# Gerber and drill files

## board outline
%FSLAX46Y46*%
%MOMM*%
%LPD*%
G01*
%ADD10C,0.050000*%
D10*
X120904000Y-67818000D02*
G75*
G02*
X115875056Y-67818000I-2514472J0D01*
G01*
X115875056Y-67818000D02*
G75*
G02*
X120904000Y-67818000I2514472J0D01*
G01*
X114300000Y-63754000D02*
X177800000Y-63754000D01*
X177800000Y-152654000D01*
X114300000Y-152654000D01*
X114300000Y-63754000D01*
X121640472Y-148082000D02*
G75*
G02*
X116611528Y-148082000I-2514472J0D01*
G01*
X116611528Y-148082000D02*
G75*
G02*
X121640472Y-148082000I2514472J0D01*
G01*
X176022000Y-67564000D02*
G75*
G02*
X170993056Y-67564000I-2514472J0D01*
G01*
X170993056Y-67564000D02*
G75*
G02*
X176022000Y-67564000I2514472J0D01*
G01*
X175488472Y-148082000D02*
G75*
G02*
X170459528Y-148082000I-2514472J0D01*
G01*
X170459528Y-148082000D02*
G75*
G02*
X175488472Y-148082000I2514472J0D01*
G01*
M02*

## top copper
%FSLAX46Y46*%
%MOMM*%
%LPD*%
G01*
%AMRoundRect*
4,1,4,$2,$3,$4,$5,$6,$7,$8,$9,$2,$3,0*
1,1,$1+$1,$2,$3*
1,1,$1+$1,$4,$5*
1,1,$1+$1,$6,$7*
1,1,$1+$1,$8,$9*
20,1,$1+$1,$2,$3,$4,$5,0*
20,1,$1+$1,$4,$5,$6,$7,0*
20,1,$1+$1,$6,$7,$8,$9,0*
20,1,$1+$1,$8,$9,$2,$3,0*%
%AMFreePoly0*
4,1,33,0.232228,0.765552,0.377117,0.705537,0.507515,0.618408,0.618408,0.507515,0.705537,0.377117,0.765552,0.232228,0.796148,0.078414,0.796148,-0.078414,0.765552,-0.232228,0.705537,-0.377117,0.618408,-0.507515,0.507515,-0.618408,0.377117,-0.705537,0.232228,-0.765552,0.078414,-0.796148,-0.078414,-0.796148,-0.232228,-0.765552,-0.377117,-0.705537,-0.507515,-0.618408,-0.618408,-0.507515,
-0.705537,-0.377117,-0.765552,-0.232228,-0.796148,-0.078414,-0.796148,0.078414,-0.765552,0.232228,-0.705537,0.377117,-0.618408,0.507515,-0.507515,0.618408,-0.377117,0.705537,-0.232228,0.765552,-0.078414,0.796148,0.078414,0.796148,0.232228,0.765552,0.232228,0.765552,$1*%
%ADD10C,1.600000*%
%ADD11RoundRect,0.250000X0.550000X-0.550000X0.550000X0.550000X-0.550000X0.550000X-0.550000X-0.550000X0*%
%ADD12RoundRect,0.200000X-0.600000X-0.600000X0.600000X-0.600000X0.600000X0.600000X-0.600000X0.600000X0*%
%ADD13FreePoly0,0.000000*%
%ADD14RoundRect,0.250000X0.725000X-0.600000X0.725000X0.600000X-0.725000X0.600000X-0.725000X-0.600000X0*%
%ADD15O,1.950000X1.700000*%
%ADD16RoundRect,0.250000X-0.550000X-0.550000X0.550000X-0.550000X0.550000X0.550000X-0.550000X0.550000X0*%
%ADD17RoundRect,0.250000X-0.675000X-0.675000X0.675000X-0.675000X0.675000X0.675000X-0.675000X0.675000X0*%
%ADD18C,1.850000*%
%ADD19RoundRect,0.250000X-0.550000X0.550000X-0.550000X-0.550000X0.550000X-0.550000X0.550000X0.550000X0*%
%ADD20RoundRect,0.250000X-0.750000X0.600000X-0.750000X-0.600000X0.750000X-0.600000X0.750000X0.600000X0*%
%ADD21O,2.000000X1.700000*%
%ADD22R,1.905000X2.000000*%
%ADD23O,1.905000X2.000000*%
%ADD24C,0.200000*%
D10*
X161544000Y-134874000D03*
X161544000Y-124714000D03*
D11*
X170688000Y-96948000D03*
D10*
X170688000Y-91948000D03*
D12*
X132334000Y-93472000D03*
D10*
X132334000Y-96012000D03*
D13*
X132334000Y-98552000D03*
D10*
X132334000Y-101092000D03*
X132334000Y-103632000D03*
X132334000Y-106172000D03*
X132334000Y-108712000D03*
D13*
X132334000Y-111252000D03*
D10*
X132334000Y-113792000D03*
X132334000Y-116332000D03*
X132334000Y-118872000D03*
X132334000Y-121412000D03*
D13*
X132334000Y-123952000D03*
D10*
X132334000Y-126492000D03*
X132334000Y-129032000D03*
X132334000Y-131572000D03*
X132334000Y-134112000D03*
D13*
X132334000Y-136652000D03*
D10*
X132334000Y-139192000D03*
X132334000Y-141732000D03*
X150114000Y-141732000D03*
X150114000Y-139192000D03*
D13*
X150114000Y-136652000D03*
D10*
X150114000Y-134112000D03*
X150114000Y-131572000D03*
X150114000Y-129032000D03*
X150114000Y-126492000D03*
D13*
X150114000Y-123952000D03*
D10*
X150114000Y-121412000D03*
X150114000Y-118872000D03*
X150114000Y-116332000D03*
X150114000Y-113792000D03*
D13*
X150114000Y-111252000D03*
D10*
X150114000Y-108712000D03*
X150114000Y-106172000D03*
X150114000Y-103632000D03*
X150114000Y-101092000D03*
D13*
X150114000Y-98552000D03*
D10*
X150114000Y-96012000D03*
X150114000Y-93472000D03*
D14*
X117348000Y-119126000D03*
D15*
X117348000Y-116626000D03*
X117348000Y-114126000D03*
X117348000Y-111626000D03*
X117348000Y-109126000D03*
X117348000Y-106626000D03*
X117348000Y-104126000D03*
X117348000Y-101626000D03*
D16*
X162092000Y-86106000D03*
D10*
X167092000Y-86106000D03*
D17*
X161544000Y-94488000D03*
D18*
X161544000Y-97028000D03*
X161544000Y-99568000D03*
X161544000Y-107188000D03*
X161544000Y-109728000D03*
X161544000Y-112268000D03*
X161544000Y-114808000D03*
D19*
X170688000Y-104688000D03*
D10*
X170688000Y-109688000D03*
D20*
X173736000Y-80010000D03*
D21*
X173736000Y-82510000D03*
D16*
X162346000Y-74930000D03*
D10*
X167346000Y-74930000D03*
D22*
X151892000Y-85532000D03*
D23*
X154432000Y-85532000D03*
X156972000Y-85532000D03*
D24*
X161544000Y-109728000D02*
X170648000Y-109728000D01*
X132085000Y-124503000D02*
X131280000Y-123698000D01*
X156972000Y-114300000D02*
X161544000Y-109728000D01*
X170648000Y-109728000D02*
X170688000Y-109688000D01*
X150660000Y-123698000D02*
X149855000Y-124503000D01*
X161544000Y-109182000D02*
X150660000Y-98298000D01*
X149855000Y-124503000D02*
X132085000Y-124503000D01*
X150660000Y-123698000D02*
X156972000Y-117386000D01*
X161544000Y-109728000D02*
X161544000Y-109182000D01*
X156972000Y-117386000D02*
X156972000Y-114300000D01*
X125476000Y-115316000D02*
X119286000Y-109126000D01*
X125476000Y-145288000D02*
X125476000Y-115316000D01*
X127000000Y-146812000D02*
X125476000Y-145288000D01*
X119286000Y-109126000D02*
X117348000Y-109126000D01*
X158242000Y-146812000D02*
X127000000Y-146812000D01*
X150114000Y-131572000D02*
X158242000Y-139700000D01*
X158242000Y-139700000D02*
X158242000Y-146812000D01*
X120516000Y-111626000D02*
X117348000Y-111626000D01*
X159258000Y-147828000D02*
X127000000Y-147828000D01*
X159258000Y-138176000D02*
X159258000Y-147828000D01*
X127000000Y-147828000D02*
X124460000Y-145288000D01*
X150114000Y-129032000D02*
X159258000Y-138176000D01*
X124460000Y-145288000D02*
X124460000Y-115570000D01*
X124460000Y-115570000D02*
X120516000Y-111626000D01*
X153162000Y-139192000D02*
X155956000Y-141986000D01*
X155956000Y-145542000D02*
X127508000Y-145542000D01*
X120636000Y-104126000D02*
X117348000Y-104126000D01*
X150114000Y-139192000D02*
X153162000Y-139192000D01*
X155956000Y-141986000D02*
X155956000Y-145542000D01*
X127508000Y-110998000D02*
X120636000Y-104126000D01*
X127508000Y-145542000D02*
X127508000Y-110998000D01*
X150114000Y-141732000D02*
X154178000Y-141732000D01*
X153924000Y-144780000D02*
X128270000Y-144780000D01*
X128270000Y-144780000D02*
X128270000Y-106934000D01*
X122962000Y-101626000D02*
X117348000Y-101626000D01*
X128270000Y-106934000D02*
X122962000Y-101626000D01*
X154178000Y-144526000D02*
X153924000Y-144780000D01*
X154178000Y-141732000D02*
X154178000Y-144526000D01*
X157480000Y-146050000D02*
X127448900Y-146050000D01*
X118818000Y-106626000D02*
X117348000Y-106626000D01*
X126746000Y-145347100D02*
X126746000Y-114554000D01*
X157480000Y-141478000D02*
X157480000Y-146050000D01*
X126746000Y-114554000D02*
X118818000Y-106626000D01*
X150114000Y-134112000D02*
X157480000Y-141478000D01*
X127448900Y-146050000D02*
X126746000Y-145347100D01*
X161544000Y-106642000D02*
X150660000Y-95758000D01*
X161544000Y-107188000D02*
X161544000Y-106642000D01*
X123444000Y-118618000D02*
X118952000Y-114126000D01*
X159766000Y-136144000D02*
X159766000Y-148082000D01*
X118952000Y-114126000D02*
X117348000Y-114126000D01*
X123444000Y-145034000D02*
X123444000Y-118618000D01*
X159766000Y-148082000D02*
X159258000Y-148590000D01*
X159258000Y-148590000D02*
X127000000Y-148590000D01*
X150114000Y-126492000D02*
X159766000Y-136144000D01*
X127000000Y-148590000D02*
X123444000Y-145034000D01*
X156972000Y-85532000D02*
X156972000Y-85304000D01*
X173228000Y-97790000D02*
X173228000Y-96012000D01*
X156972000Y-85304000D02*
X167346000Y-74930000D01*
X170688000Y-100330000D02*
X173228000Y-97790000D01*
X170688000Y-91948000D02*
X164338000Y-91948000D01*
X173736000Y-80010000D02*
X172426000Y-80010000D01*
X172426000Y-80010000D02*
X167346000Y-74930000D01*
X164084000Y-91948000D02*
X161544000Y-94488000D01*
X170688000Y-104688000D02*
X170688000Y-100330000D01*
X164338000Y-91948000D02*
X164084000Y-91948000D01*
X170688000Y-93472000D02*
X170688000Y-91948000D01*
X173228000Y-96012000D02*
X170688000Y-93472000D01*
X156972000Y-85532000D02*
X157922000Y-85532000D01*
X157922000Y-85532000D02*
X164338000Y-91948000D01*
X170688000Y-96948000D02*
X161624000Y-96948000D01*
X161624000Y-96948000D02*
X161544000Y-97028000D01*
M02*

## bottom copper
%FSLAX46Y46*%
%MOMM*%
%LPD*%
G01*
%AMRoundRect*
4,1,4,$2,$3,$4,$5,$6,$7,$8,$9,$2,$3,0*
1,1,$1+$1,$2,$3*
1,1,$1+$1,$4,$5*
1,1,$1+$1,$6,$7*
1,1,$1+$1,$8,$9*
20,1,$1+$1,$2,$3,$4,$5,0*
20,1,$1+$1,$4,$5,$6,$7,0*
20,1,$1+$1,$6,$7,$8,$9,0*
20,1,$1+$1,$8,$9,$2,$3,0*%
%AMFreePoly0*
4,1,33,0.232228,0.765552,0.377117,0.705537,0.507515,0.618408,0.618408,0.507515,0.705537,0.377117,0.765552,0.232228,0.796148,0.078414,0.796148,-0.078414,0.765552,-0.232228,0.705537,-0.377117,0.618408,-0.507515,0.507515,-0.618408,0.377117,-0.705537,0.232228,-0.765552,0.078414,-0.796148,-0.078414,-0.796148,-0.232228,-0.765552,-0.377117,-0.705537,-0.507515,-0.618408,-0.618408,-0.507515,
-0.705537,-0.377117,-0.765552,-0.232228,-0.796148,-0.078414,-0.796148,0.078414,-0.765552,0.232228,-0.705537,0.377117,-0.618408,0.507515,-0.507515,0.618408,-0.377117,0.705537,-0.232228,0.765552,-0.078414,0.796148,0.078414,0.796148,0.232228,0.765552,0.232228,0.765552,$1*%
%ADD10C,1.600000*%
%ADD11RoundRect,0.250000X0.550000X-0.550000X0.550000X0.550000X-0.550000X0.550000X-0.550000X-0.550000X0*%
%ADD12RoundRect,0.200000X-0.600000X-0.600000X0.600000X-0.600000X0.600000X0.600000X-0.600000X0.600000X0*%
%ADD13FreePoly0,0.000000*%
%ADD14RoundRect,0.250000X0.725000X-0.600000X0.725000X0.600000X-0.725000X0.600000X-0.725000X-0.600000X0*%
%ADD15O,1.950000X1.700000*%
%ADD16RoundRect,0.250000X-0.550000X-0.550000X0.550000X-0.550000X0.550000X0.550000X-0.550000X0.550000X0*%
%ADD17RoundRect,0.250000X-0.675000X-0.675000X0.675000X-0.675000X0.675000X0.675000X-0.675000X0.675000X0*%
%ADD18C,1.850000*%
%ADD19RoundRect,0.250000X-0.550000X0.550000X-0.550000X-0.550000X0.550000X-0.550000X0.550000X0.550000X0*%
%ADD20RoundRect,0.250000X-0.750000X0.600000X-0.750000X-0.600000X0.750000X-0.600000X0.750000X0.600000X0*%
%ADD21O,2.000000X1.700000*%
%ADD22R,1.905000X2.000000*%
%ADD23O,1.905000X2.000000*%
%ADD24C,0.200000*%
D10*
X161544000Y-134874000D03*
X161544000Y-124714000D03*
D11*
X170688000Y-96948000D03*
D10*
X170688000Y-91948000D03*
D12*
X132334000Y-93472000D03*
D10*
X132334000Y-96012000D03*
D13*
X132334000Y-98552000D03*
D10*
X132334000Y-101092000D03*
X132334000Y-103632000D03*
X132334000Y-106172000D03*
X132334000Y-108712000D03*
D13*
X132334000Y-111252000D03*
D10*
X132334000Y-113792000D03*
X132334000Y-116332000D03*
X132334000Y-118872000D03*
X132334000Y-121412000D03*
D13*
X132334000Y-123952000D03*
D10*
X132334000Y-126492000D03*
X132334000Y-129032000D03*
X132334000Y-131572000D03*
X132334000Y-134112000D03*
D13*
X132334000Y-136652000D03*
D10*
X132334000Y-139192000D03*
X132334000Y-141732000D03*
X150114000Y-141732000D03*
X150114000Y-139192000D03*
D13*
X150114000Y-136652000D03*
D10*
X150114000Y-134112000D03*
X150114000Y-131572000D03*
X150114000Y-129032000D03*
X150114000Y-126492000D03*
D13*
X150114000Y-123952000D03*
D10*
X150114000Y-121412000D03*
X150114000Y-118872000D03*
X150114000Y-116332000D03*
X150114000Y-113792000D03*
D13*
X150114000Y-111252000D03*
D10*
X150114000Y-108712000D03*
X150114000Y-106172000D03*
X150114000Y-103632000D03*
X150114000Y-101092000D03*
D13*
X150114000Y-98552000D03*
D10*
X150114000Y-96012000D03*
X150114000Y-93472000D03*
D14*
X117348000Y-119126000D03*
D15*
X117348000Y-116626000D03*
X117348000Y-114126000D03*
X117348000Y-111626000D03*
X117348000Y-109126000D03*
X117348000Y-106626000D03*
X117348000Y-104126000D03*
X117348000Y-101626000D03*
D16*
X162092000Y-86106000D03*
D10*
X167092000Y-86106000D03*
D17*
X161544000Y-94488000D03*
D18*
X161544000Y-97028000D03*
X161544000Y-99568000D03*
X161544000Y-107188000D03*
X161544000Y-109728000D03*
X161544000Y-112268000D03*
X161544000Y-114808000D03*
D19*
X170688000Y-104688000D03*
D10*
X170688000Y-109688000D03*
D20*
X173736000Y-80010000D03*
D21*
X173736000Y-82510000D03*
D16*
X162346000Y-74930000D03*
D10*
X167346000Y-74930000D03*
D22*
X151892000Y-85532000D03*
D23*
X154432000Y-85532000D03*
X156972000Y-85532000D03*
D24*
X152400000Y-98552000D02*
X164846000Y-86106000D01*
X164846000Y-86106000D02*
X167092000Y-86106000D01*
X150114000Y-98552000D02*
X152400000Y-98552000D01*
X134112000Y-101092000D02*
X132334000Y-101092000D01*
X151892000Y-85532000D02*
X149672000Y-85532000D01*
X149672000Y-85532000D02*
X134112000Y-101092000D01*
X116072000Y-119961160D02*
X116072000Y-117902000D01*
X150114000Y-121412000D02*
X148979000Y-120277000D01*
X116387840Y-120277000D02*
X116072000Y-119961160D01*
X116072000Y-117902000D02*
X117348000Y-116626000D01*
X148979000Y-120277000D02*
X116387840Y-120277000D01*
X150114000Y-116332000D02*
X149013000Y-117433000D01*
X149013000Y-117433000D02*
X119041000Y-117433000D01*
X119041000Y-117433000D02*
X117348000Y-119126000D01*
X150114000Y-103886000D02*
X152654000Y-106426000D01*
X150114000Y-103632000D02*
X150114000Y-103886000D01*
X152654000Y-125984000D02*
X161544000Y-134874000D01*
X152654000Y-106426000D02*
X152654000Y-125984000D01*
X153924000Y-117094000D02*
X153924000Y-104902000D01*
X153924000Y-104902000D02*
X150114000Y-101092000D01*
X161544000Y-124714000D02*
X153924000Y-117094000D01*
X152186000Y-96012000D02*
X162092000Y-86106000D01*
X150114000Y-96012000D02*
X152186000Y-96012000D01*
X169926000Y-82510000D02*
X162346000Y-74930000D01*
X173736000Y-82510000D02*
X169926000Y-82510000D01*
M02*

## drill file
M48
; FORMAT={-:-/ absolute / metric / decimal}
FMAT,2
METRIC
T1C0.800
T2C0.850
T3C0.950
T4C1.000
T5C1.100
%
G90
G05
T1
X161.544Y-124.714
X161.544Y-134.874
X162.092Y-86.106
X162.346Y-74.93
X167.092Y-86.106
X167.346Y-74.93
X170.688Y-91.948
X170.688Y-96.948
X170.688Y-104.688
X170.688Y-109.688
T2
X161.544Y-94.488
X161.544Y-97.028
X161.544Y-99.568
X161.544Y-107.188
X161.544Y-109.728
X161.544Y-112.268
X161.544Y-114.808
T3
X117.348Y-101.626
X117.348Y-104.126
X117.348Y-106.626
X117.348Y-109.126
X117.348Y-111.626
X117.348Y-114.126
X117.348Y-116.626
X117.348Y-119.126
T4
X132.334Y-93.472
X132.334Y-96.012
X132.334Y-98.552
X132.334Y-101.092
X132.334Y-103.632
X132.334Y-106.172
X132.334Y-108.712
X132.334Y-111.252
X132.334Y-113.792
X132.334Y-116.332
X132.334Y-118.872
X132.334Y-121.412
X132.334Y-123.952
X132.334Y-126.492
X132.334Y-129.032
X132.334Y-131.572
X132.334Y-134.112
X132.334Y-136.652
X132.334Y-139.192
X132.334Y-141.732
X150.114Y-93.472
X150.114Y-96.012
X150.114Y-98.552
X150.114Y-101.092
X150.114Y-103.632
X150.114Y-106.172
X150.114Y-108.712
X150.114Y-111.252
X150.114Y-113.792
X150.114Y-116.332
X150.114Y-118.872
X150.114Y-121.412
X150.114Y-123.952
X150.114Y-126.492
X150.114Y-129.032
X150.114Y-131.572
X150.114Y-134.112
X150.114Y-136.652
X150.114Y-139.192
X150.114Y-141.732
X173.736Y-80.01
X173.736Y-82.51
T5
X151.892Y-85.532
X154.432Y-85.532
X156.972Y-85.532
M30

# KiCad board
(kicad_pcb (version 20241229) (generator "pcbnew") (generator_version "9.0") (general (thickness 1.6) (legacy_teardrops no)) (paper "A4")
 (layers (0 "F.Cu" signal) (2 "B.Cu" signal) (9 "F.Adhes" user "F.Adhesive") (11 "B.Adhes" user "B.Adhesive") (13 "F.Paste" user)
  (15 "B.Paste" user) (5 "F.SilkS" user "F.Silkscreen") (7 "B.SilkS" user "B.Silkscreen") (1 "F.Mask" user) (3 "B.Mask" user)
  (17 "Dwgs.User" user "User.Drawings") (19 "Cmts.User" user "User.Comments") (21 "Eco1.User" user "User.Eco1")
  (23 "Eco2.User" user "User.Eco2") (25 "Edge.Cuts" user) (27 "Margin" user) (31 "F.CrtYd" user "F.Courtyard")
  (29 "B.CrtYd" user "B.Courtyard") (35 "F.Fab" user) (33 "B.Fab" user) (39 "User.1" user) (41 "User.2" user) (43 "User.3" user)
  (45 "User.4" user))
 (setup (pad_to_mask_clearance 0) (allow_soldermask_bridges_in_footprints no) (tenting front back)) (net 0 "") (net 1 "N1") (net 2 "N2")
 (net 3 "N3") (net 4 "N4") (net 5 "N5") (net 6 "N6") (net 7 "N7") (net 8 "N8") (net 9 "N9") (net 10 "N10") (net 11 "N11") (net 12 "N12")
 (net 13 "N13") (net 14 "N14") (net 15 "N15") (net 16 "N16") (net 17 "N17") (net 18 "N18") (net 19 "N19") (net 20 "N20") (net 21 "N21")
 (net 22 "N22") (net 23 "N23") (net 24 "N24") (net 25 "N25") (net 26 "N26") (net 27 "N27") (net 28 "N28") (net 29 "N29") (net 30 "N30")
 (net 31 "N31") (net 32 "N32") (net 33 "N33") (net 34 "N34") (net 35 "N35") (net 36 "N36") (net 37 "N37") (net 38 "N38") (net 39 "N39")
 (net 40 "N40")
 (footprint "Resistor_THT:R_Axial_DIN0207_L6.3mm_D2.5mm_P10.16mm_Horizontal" (layer "F.Cu") (at 161.544 134.874 90)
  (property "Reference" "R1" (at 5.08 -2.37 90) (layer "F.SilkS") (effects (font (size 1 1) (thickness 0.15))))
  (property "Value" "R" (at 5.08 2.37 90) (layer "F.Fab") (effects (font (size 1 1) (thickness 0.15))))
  (pad "1" thru_hole circle (at 0 0 90) (size 1.6 1.6) (drill 0.8) (layers "*.Cu" "*.Mask") (remove_unused_layers no) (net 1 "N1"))
  (pad "2" thru_hole circle (at 10.16 0 90) (size 1.6 1.6) (drill 0.8) (layers "*.Cu" "*.Mask") (remove_unused_layers no) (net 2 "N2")))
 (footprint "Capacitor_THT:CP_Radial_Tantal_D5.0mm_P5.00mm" (layer "F.Cu") (at 170.688 96.948 90)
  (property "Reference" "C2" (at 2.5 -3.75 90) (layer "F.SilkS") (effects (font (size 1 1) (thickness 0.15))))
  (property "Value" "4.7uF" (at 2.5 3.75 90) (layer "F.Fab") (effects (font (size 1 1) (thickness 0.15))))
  (pad "1" thru_hole roundrect (at 0 0 90) (size 1.6 1.6) (drill 0.8) (layers "*.Cu" "*.Mask") (remove_unused_layers no)
   (roundrect_rratio 0.15625) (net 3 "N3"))
  (pad "2" thru_hole circle (at 5 0 90) (size 1.6 1.6) (drill 0.8) (layers "*.Cu" "*.Mask") (remove_unused_layers no) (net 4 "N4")))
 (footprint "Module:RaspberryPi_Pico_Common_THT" (layer "F.Cu") (at 132.334 93.472)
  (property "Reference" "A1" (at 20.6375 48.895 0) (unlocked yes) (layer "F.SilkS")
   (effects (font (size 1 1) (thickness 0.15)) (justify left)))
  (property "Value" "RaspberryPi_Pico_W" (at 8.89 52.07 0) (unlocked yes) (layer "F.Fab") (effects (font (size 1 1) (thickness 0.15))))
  (pad "1" thru_hole roundrect (at 0 0) (size 1.6 1.6) (drill 1) (layers "*.Cu" "*.Mask") (remove_unused_layers no) (roundrect_rratio 0.125)
   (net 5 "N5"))
  (pad "2" thru_hole circle (at 0 2.54) (size 1.6 1.6) (drill 1) (layers "*.Cu" "*.Mask") (remove_unused_layers no) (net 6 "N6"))
  (pad "3" thru_hole custom (at 0 5.08) (size 1.6 1.6) (drill 1) (layers "*.Cu" "*.Mask") (remove_unused_layers no) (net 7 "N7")
   (options (clearance outline) (anchor circle)) (primitives))
  (pad "4" thru_hole circle (at 0 7.62) (size 1.6 1.6) (drill 1) (layers "*.Cu" "*.Mask") (remove_unused_layers no) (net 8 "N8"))
  (pad "5" thru_hole circle (at 0 10.16) (size 1.6 1.6) (drill 1) (layers "*.Cu" "*.Mask") (remove_unused_layers no) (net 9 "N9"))
  (pad "6" thru_hole circle (at 0 12.7) (size 1.6 1.6) (drill 1) (layers "*.Cu" "*.Mask") (remove_unused_layers no) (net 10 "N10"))
  (pad "7" thru_hole circle (at 0 15.24) (size 1.6 1.6) (drill 1) (layers "*.Cu" "*.Mask") (remove_unused_layers no) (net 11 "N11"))
  (pad "8" thru_hole custom (at 0 17.78) (size 1.6 1.6) (drill 1) (layers "*.Cu" "*.Mask") (remove_unused_layers no) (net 7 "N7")
   (options (clearance outline) (anchor circle)) (primitives))
  (pad "9" thru_hole circle (at 0 20.32) (size 1.6 1.6) (drill 1) (layers "*.Cu" "*.Mask") (remove_unused_layers no) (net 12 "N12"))
  (pad "10" thru_hole circle (at 0 22.86) (size 1.6 1.6) (drill 1) (layers "*.Cu" "*.Mask") (remove_unused_layers no) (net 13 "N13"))
  (pad "11" thru_hole circle (at 0 25.4) (size 1.6 1.6) (drill 1) (layers "*.Cu" "*.Mask") (remove_unused_layers no) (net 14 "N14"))
  (pad "12" thru_hole circle (at 0 27.94) (size 1.6 1.6) (drill 1) (layers "*.Cu" "*.Mask") (remove_unused_layers no) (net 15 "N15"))
  (pad "13" thru_hole custom (at 0 30.48) (size 1.6 1.6) (drill 1) (layers "*.Cu" "*.Mask") (remove_unused_layers no) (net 7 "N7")
   (options (clearance outline) (anchor circle)) (primitives))
  (pad "14" thru_hole circle (at 0 33.02) (size 1.6 1.6) (drill 1) (layers "*.Cu" "*.Mask") (remove_unused_layers no) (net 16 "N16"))
  (pad "15" thru_hole circle (at 0 35.56) (size 1.6 1.6) (drill 1) (layers "*.Cu" "*.Mask") (remove_unused_layers no) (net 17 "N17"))
  (pad "16" thru_hole circle (at 0 38.1) (size 1.6 1.6) (drill 1) (layers "*.Cu" "*.Mask") (remove_unused_layers no) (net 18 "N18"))
  (pad "17" thru_hole circle (at 0 40.64) (size 1.6 1.6) (drill 1) (layers "*.Cu" "*.Mask") (remove_unused_layers no) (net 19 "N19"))
  (pad "18" thru_hole custom (at 0 43.18) (size 1.6 1.6) (drill 1) (layers "*.Cu" "*.Mask") (remove_unused_layers no) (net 7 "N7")
   (options (clearance outline) (anchor circle)) (primitives))
  (pad "19" thru_hole circle (at 0 45.72) (size 1.6 1.6) (drill 1) (layers "*.Cu" "*.Mask") (remove_unused_layers no) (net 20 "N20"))
  (pad "20" thru_hole circle (at 0 48.26) (size 1.6 1.6) (drill 1) (layers "*.Cu" "*.Mask") (remove_unused_layers no) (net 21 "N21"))
  (pad "21" thru_hole circle (at 17.78 48.26) (size 1.6 1.6) (drill 1) (layers "*.Cu" "*.Mask") (remove_unused_layers no) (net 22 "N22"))
  (pad "22" thru_hole circle (at 17.78 45.72) (size 1.6 1.6) (drill 1) (layers "*.Cu" "*.Mask") (remove_unused_layers no) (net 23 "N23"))
  (pad "23" thru_hole custom (at 17.78 43.18) (size 1.6 1.6) (drill 1) (layers "*.Cu" "*.Mask") (remove_unused_layers no) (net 7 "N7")
   (options (clearance outline) (anchor circle)) (primitives))
  (pad "24" thru_hole circle (at 17.78 40.64) (size 1.6 1.6) (drill 1) (layers "*.Cu" "*.Mask") (remove_unused_layers no) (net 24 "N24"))
  (pad "25" thru_hole circle (at 17.78 38.1) (size 1.6 1.6) (drill 1) (layers "*.Cu" "*.Mask") (remove_unused_layers no) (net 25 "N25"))
  (pad "26" thru_hole circle (at 17.78 35.56) (size 1.6 1.6) (drill 1) (layers "*.Cu" "*.Mask") (remove_unused_layers no) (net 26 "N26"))
  (pad "27" thru_hole circle (at 17.78 33.02) (size 1.6 1.6) (drill 1) (layers "*.Cu" "*.Mask") (remove_unused_layers no) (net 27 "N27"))
  (pad "28" thru_hole custom (at 17.78 30.48) (size 1.6 1.6) (drill 1) (layers "*.Cu" "*.Mask") (remove_unused_layers no) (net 7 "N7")
   (options (clearance outline) (anchor circle)) (primitives))
  (pad "29" thru_hole circle (at 17.78 27.94) (size 1.6 1.6) (drill 1) (layers "*.Cu" "*.Mask") (remove_unused_layers no) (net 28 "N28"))
  (pad "30" thru_hole circle (at 17.78 25.4) (size 1.6 1.6) (drill 1) (layers "*.Cu" "*.Mask") (remove_unused_layers no) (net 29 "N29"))
  (pad "31" thru_hole circle (at 17.78 22.86) (size 1.6 1.6) (drill 1) (layers "*.Cu" "*.Mask") (remove_unused_layers no) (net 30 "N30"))
  (pad "32" thru_hole circle (at 17.78 20.32) (size 1.6 1.6) (drill 1) (layers "*.Cu" "*.Mask") (remove_unused_layers no) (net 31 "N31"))
  (pad "33" thru_hole custom (at 17.78 17.78) (size 1.6 1.6) (drill 1) (layers "*.Cu" "*.Mask") (remove_unused_layers no) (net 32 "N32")
   (options (clearance outline) (anchor circle)) (primitives))
  (pad "34" thru_hole circle (at 17.78 15.24) (size 1.6 1.6) (drill 1) (layers "*.Cu" "*.Mask") (remove_unused_layers no) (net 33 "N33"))
  (pad "35" thru_hole circle (at 17.78 12.7) (size 1.6 1.6) (drill 1) (layers "*.Cu" "*.Mask") (remove_unused_layers no) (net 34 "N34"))
  (pad "36" thru_hole circle (at 17.78 10.16) (size 1.6 1.6) (drill 1) (layers "*.Cu" "*.Mask") (remove_unused_layers no) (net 1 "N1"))
  (pad "37" thru_hole circle (at 17.78 7.62) (size 1.6 1.6) (drill 1) (layers "*.Cu" "*.Mask") (remove_unused_layers no) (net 2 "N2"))
  (pad "38" thru_hole custom (at 17.78 5.08) (size 1.6 1.6) (drill 1) (layers "*.Cu" "*.Mask") (remove_unused_layers no) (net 7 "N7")
   (options (clearance outline) (anchor circle)) (primitives))
  (pad "39" thru_hole circle (at 17.78 2.54) (size 1.6 1.6) (drill 1) (layers "*.Cu" "*.Mask") (remove_unused_layers no) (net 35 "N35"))
  (pad "40" thru_hole circle (at 17.78 0) (size 1.6 1.6) (drill 1) (layers "*.Cu" "*.Mask") (remove_unused_layers no) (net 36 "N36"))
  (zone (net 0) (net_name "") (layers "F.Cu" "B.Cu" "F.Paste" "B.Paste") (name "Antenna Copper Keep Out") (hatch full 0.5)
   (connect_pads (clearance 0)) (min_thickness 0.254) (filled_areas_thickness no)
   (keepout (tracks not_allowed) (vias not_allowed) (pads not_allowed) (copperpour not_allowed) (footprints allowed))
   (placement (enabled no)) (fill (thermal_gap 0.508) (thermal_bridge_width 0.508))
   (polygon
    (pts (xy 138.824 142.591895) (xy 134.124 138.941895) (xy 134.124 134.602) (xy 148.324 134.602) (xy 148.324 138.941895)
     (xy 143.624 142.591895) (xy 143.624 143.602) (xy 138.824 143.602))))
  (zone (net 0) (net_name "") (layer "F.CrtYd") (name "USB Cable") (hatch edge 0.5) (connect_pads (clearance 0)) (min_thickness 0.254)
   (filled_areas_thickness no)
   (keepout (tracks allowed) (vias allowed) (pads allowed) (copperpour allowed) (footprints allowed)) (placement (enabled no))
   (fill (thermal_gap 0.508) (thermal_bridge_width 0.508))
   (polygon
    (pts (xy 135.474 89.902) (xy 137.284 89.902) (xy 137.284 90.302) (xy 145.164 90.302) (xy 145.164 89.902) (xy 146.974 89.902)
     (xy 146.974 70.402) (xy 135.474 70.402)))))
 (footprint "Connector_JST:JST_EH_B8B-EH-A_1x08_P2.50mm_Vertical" (layer "F.Cu") (at 117.348 119.126 90)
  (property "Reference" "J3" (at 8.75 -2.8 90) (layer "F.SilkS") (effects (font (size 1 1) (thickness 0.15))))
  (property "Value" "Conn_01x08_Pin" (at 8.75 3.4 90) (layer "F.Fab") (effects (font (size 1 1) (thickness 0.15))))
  (pad "1" thru_hole roundrect (at 0 0 90) (size 1.7 1.95) (drill 0.95) (layers "*.Cu" "*.Mask") (remove_unused_layers no)
   (roundrect_rratio 0.147059) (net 30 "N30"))
  (pad "2" thru_hole oval (at 2.5 0 90) (size 1.7 1.95) (drill 0.95) (layers "*.Cu" "*.Mask") (remove_unused_layers no) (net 28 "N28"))
  (pad "3" thru_hole oval (at 5 0 90) (size 1.7 1.95) (drill 0.95) (layers "*.Cu" "*.Mask") (remove_unused_layers no) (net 27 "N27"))
  (pad "4" thru_hole oval (at 7.5 0 90) (size 1.7 1.95) (drill 0.95) (layers "*.Cu" "*.Mask") (remove_unused_layers no) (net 26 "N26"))
  (pad "5" thru_hole oval (at 10 0 90) (size 1.7 1.95) (drill 0.95) (layers "*.Cu" "*.Mask") (remove_unused_layers no) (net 25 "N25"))
  (pad "6" thru_hole oval (at 12.5 0 90) (size 1.7 1.95) (drill 0.95) (layers "*.Cu" "*.Mask") (remove_unused_layers no) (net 24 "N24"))
  (pad "7" thru_hole oval (at 15 0 90) (size 1.7 1.95) (drill 0.95) (layers "*.Cu" "*.Mask") (remove_unused_layers no) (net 23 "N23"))
  (pad "8" thru_hole oval (at 17.5 0 90) (size 1.7 1.95) (drill 0.95) (layers "*.Cu" "*.Mask") (remove_unused_layers no) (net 22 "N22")))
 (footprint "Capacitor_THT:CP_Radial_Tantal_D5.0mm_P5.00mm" (layer "F.Cu") (at 162.092 86.106)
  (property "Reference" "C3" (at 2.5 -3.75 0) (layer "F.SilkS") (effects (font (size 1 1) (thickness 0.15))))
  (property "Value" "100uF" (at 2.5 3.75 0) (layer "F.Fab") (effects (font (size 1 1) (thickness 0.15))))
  (pad "1" thru_hole roundrect (at 0 0) (size 1.6 1.6) (drill 0.8) (layers "*.Cu" "*.Mask") (remove_unused_layers no)
   (roundrect_rratio 0.15625) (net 35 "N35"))
  (pad "2" thru_hole circle (at 5 0) (size 1.6 1.6) (drill 0.8) (layers "*.Cu" "*.Mask") (remove_unused_layers no) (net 7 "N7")))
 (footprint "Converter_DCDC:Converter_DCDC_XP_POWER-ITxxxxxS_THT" (layer "F.Cu") (at 161.544 94.488)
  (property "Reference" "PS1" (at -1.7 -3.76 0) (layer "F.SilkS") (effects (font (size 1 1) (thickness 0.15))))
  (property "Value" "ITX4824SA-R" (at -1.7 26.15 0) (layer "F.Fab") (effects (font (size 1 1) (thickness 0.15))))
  (pad "1" thru_hole roundrect (at 0 0) (size 1.85 1.85) (drill 0.85) (layers "*.Cu" "*.Mask") (remove_unused_layers no)
   (roundrect_rratio 0.135135) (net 4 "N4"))
  (pad "2" thru_hole circle (at 0 2.54) (size 1.85 1.85) (drill 0.85) (layers "*.Cu" "*.Mask") (remove_unused_layers no) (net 3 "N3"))
  (pad "3" thru_hole circle (at 0 5.08) (size 1.85 1.85) (drill 0.85) (layers "*.Cu" "*.Mask") (remove_unused_layers no) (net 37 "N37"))
  (pad "6" thru_hole circle (at 0 12.7) (size 1.85 1.85) (drill 0.85) (layers "*.Cu" "*.Mask") (remove_unused_layers no) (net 35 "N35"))
  (pad "7" thru_hole circle (at 0 15.24) (size 1.85 1.85) (drill 0.85) (layers "*.Cu" "*.Mask") (remove_unused_layers no) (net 7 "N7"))
  (pad "8" thru_hole circle (at 0 17.78) (size 1.85 1.85) (drill 0.85) (layers "*.Cu" "*.Mask") (remove_unused_layers no) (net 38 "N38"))
  (pad "9" thru_hole circle (at 0 20.32) (size 1.85 1.85) (drill 0.85) (layers "*.Cu" "*.Mask") (remove_unused_layers no)))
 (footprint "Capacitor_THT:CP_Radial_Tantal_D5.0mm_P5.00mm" (layer "F.Cu") (at 170.688 104.688 -90)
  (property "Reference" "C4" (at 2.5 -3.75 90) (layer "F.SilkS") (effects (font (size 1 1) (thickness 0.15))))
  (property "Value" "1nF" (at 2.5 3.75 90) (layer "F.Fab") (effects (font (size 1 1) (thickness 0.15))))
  (pad "1" thru_hole roundrect (at 0 0 270) (size 1.6 1.6) (drill 0.8) (layers "*.Cu" "*.Mask") (remove_unused_layers no)
   (roundrect_rratio 0.15625) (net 4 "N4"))
  (pad "2" thru_hole circle (at 5 0 270) (size 1.6 1.6) (drill 0.8) (layers "*.Cu" "*.Mask") (remove_unused_layers no) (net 7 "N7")))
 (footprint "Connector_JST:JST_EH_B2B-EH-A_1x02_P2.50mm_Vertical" (layer "F.Cu") (at 173.736 80.01 -90)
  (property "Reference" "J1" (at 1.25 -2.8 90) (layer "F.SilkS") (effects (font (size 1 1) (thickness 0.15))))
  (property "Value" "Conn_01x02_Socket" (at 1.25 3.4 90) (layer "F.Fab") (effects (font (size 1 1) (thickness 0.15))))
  (pad "1" thru_hole roundrect (at 0 0 270) (size 1.7 2) (drill 1) (layers "*.Cu" "*.Mask") (remove_unused_layers no)
   (roundrect_rratio 0.147059) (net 4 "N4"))
  (pad "2" thru_hole oval (at 2.5 0 270) (size 1.7 2) (drill 1) (layers "*.Cu" "*.Mask") (remove_unused_layers no) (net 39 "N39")))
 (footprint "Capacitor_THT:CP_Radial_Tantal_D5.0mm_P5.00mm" (layer "F.Cu") (at 162.346 74.93)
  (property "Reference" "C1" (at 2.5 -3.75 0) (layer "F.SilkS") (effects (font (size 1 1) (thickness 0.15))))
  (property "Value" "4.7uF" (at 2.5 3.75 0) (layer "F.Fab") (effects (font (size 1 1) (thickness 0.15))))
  (pad "1" thru_hole roundrect (at 0 0) (size 1.6 1.6) (drill 0.8) (layers "*.Cu" "*.Mask") (remove_unused_layers no)
   (roundrect_rratio 0.15625) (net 39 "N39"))
  (pad "2" thru_hole circle (at 5 0) (size 1.6 1.6) (drill 0.8) (layers "*.Cu" "*.Mask") (remove_unused_layers no) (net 4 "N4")))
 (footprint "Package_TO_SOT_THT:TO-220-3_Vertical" (layer "F.Cu") (at 151.892 85.532)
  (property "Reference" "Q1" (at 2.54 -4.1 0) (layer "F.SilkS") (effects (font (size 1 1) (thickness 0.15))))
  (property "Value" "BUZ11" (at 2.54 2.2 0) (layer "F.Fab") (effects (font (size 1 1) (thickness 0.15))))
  (pad "1" thru_hole rect (at 0 0) (size 1.905 2) (drill 1.1) (layers "*.Cu" "*.Mask") (remove_unused_layers no) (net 8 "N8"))
  (pad "2" thru_hole oval (at 2.54 0) (size 1.905 2) (drill 1.1) (layers "*.Cu" "*.Mask") (remove_unused_layers no) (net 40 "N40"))
  (pad "3" thru_hole oval (at 5.08 0) (size 1.905 2) (drill 1.1) (layers "*.Cu" "*.Mask") (remove_unused_layers no) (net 4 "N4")))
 (gr_circle (center 118.389528 67.818) (end 120.167528 69.596) (stroke (width 0.05) (type default)) (fill no) (layer "Edge.Cuts"))
 (gr_rect (start 114.3 63.754) (end 177.8 152.654) (stroke (width 0.05) (type default)) (fill no) (layer "Edge.Cuts"))
 (gr_circle (center 119.126 148.082) (end 120.904 149.86) (stroke (width 0.05) (type default)) (fill no) (layer "Edge.Cuts"))
 (gr_circle (center 173.507528 67.564) (end 175.285528 69.342) (stroke (width 0.05) (type default)) (fill no) (layer "Edge.Cuts"))
 (gr_circle (center 172.974 148.082) (end 174.752 149.86) (stroke (width 0.05) (type default)) (fill no) (layer "Edge.Cuts"))
 (segment (start 161.544 109.728) (end 170.648 109.728) (width 0.2) (layer "F.Cu") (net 7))
 (segment (start 132.085 124.503) (end 131.28 123.698) (width 0.2) (layer "F.Cu") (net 7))
 (segment (start 156.972 114.3) (end 161.544 109.728) (width 0.2) (layer "F.Cu") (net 7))
 (segment (start 170.648 109.728) (end 170.688 109.688) (width 0.2) (layer "F.Cu") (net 7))
 (segment (start 150.66 123.698) (end 149.855 124.503) (width 0.2) (layer "F.Cu") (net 7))
 (segment (start 161.544 109.182) (end 150.66 98.298) (width 0.2) (layer "F.Cu") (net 7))
 (segment (start 149.855 124.503) (end 132.085 124.503) (width 0.2) (layer "F.Cu") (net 7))
 (segment (start 150.66 123.698) (end 156.972 117.386) (width 0.2) (layer "F.Cu") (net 7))
 (segment (start 161.544 109.728) (end 161.544 109.182) (width 0.2) (layer "F.Cu") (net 7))
 (segment (start 156.972 117.386) (end 156.972 114.3) (width 0.2) (layer "F.Cu") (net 7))
 (segment (start 152.4 98.552) (end 164.846 86.106) (width 0.2) (layer "B.Cu") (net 7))
 (segment (start 164.846 86.106) (end 167.092 86.106) (width 0.2) (layer "B.Cu") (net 7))
 (segment (start 150.114 98.552) (end 152.4 98.552) (width 0.2) (layer "B.Cu") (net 7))
 (segment (start 134.112 101.092) (end 132.334 101.092) (width 0.2) (layer "B.Cu") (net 8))
 (segment (start 151.892 85.532) (end 149.672 85.532) (width 0.2) (layer "B.Cu") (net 8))
 (segment (start 149.672 85.532) (end 134.112 101.092) (width 0.2) (layer "B.Cu") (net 8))
 (segment (start 125.476 115.316) (end 119.286 109.126) (width 0.2) (layer "F.Cu") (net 25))
 (segment (start 125.476 145.288) (end 125.476 115.316) (width 0.2) (layer "F.Cu") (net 25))
 (segment (start 127 146.812) (end 125.476 145.288) (width 0.2) (layer "F.Cu") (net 25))
 (segment (start 119.286 109.126) (end 117.348 109.126) (width 0.2) (layer "F.Cu") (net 25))
 (segment (start 158.242 146.812) (end 127 146.812) (width 0.2) (layer "F.Cu") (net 25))
 (segment (start 150.114 131.572) (end 158.242 139.7) (width 0.2) (layer "F.Cu") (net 25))
 (segment (start 158.242 139.7) (end 158.242 146.812) (width 0.2) (layer "F.Cu") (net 25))
 (segment (start 116.072 119.96116) (end 116.072 117.902) (width 0.2) (layer "B.Cu") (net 28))
 (segment (start 150.114 121.412) (end 148.979 120.277) (width 0.2) (layer "B.Cu") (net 28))
 (segment (start 116.38784 120.277) (end 116.072 119.96116) (width 0.2) (layer "B.Cu") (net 28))
 (segment (start 116.072 117.902) (end 117.348 116.626) (width 0.2) (layer "B.Cu") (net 28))
 (segment (start 148.979 120.277) (end 116.38784 120.277) (width 0.2) (layer "B.Cu") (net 28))
 (segment (start 120.516 111.626) (end 117.348 111.626) (width 0.2) (layer "F.Cu") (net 26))
 (segment (start 159.258 147.828) (end 127 147.828) (width 0.2) (layer "F.Cu") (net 26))
 (segment (start 159.258 138.176) (end 159.258 147.828) (width 0.2) (layer "F.Cu") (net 26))
 (segment (start 127 147.828) (end 124.46 145.288) (width 0.2) (layer "F.Cu") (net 26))
 (segment (start 150.114 129.032) (end 159.258 138.176) (width 0.2) (layer "F.Cu") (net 26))
 (segment (start 124.46 145.288) (end 124.46 115.57) (width 0.2) (layer "F.Cu") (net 26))
 (segment (start 124.46 115.57) (end 120.516 111.626) (width 0.2) (layer "F.Cu") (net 26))
 (segment (start 150.114 116.332) (end 149.013 117.433) (width 0.2) (layer "B.Cu") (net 30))
 (segment (start 149.013 117.433) (end 119.041 117.433) (width 0.2) (layer "B.Cu") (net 30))
 (segment (start 119.041 117.433) (end 117.348 119.126) (width 0.2) (layer "B.Cu") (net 30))
 (segment (start 150.114 103.886) (end 152.654 106.426) (width 0.2) (layer "B.Cu") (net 1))
 (segment (start 150.114 103.632) (end 150.114 103.886) (width 0.2) (layer "B.Cu") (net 1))
 (segment (start 152.654 125.984) (end 161.544 134.874) (width 0.2) (layer "B.Cu") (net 1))
 (segment (start 152.654 106.426) (end 152.654 125.984) (width 0.2) (layer "B.Cu") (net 1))
 (segment (start 153.162 139.192) (end 155.956 141.986) (width 0.2) (layer "F.Cu") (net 23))
 (segment (start 155.956 145.542) (end 127.508 145.542) (width 0.2) (layer "F.Cu") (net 23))
 (segment (start 120.636 104.126) (end 117.348 104.126) (width 0.2) (layer "F.Cu") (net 23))
 (segment (start 150.114 139.192) (end 153.162 139.192) (width 0.2) (layer "F.Cu") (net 23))
 (segment (start 155.956 141.986) (end 155.956 145.542) (width 0.2) (layer "F.Cu") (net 23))
 (segment (start 127.508 110.998) (end 120.636 104.126) (width 0.2) (layer "F.Cu") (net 23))
 (segment (start 127.508 145.542) (end 127.508 110.998) (width 0.2) (layer "F.Cu") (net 23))
 (segment (start 153.924 117.094) (end 153.924 104.902) (width 0.2) (layer "B.Cu") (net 2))
 (segment (start 153.924 104.902) (end 150.114 101.092) (width 0.2) (layer "B.Cu") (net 2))
 (segment (start 161.544 124.714) (end 153.924 117.094) (width 0.2) (layer "B.Cu") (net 2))
 (segment (start 150.114 141.732) (end 154.178 141.732) (width 0.2) (layer "F.Cu") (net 22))
 (segment (start 153.924 144.78) (end 128.27 144.78) (width 0.2) (layer "F.Cu") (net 22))
 (segment (start 128.27 144.78) (end 128.27 106.934) (width 0.2) (layer "F.Cu") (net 22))
 (segment (start 122.962 101.626) (end 117.348 101.626) (width 0.2) (layer "F.Cu") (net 22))
 (segment (start 128.27 106.934) (end 122.962 101.626) (width 0.2) (layer "F.Cu") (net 22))
 (segment (start 154.178 144.526) (end 153.924 144.78) (width 0.2) (layer "F.Cu") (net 22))
 (segment (start 154.178 141.732) (end 154.178 144.526) (width 0.2) (layer "F.Cu") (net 22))
 (segment (start 157.48 146.05) (end 127.4489 146.05) (width 0.2) (layer "F.Cu") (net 24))
 (segment (start 118.818 106.626) (end 117.348 106.626) (width 0.2) (layer "F.Cu") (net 24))
 (segment (start 126.746 145.3471) (end 126.746 114.554) (width 0.2) (layer "F.Cu") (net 24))
 (segment (start 157.48 141.478) (end 157.48 146.05) (width 0.2) (layer "F.Cu") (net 24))
 (segment (start 126.746 114.554) (end 118.818 106.626) (width 0.2) (layer "F.Cu") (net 24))
 (segment (start 150.114 134.112) (end 157.48 141.478) (width 0.2) (layer "F.Cu") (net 24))
 (segment (start 127.4489 146.05) (end 126.746 145.3471) (width 0.2) (layer "F.Cu") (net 24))
 (segment (start 161.544 106.642) (end 150.66 95.758) (width 0.2) (layer "F.Cu") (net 35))
 (segment (start 161.544 107.188) (end 161.544 106.642) (width 0.2) (layer "F.Cu") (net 35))
 (segment (start 152.186 96.012) (end 162.092 86.106) (width 0.2) (layer "B.Cu") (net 35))
 (segment (start 150.114 96.012) (end 152.186 96.012) (width 0.2) (layer "B.Cu") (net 35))
 (segment (start 123.444 118.618) (end 118.952 114.126) (width 0.2) (layer "F.Cu") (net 27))
 (segment (start 159.766 136.144) (end 159.766 148.082) (width 0.2) (layer "F.Cu") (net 27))
 (segment (start 118.952 114.126) (end 117.348 114.126) (width 0.2) (layer "F.Cu") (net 27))
 (segment (start 123.444 145.034) (end 123.444 118.618) (width 0.2) (layer "F.Cu") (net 27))
 (segment (start 159.766 148.082) (end 159.258 148.59) (width 0.2) (layer "F.Cu") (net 27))
 (segment (start 159.258 148.59) (end 127 148.59) (width 0.2) (layer "F.Cu") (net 27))
 (segment (start 150.114 126.492) (end 159.766 136.144) (width 0.2) (layer "F.Cu") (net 27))
 (segment (start 127 148.59) (end 123.444 145.034) (width 0.2) (layer "F.Cu") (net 27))
 (segment (start 156.972 85.532) (end 156.972 85.304) (width 0.2) (layer "F.Cu") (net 4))
 (segment (start 173.228 97.79) (end 173.228 96.012) (width 0.2) (layer "F.Cu") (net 4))
 (segment (start 156.972 85.304) (end 167.346 74.93) (width 0.2) (layer "F.Cu") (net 4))
 (segment (start 170.688 100.33) (end 173.228 97.79) (width 0.2) (layer "F.Cu") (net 4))
 (segment (start 170.688 91.948) (end 164.338 91.948) (width 0.2) (layer "F.Cu") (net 4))
 (segment (start 173.736 80.01) (end 172.426 80.01) (width 0.2) (layer "F.Cu") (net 4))
 (segment (start 172.426 80.01) (end 167.346 74.93) (width 0.2) (layer "F.Cu") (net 4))
 (segment (start 164.084 91.948) (end 161.544 94.488) (width 0.2) (layer "F.Cu") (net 4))
 (segment (start 170.688 104.688) (end 170.688 100.33) (width 0.2) (layer "F.Cu") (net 4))
 (segment (start 164.338 91.948) (end 164.084 91.948) (width 0.2) (layer "F.Cu") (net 4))
 (segment (start 170.688 93.472) (end 170.688 91.948) (width 0.2) (layer "F.Cu") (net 4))
 (segment (start 173.228 96.012) (end 170.688 93.472) (width 0.2) (layer "F.Cu") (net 4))
 (segment (start 156.972 85.532) (end 157.922 85.532) (width 0.2) (layer "F.Cu") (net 4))
 (segment (start 157.922 85.532) (end 164.338 91.948) (width 0.2) (layer "F.Cu") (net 4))
 (segment (start 169.926 82.51) (end 162.346 74.93) (width 0.2) (layer "B.Cu") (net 39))
 (segment (start 173.736 82.51) (end 169.926 82.51) (width 0.2) (layer "B.Cu") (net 39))
 (segment (start 170.688 96.948) (end 161.624 96.948) (width 0.2) (layer "F.Cu") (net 3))
 (segment (start 161.624 96.948) (end 161.544 97.028) (width 0.2) (layer "F.Cu") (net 3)))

